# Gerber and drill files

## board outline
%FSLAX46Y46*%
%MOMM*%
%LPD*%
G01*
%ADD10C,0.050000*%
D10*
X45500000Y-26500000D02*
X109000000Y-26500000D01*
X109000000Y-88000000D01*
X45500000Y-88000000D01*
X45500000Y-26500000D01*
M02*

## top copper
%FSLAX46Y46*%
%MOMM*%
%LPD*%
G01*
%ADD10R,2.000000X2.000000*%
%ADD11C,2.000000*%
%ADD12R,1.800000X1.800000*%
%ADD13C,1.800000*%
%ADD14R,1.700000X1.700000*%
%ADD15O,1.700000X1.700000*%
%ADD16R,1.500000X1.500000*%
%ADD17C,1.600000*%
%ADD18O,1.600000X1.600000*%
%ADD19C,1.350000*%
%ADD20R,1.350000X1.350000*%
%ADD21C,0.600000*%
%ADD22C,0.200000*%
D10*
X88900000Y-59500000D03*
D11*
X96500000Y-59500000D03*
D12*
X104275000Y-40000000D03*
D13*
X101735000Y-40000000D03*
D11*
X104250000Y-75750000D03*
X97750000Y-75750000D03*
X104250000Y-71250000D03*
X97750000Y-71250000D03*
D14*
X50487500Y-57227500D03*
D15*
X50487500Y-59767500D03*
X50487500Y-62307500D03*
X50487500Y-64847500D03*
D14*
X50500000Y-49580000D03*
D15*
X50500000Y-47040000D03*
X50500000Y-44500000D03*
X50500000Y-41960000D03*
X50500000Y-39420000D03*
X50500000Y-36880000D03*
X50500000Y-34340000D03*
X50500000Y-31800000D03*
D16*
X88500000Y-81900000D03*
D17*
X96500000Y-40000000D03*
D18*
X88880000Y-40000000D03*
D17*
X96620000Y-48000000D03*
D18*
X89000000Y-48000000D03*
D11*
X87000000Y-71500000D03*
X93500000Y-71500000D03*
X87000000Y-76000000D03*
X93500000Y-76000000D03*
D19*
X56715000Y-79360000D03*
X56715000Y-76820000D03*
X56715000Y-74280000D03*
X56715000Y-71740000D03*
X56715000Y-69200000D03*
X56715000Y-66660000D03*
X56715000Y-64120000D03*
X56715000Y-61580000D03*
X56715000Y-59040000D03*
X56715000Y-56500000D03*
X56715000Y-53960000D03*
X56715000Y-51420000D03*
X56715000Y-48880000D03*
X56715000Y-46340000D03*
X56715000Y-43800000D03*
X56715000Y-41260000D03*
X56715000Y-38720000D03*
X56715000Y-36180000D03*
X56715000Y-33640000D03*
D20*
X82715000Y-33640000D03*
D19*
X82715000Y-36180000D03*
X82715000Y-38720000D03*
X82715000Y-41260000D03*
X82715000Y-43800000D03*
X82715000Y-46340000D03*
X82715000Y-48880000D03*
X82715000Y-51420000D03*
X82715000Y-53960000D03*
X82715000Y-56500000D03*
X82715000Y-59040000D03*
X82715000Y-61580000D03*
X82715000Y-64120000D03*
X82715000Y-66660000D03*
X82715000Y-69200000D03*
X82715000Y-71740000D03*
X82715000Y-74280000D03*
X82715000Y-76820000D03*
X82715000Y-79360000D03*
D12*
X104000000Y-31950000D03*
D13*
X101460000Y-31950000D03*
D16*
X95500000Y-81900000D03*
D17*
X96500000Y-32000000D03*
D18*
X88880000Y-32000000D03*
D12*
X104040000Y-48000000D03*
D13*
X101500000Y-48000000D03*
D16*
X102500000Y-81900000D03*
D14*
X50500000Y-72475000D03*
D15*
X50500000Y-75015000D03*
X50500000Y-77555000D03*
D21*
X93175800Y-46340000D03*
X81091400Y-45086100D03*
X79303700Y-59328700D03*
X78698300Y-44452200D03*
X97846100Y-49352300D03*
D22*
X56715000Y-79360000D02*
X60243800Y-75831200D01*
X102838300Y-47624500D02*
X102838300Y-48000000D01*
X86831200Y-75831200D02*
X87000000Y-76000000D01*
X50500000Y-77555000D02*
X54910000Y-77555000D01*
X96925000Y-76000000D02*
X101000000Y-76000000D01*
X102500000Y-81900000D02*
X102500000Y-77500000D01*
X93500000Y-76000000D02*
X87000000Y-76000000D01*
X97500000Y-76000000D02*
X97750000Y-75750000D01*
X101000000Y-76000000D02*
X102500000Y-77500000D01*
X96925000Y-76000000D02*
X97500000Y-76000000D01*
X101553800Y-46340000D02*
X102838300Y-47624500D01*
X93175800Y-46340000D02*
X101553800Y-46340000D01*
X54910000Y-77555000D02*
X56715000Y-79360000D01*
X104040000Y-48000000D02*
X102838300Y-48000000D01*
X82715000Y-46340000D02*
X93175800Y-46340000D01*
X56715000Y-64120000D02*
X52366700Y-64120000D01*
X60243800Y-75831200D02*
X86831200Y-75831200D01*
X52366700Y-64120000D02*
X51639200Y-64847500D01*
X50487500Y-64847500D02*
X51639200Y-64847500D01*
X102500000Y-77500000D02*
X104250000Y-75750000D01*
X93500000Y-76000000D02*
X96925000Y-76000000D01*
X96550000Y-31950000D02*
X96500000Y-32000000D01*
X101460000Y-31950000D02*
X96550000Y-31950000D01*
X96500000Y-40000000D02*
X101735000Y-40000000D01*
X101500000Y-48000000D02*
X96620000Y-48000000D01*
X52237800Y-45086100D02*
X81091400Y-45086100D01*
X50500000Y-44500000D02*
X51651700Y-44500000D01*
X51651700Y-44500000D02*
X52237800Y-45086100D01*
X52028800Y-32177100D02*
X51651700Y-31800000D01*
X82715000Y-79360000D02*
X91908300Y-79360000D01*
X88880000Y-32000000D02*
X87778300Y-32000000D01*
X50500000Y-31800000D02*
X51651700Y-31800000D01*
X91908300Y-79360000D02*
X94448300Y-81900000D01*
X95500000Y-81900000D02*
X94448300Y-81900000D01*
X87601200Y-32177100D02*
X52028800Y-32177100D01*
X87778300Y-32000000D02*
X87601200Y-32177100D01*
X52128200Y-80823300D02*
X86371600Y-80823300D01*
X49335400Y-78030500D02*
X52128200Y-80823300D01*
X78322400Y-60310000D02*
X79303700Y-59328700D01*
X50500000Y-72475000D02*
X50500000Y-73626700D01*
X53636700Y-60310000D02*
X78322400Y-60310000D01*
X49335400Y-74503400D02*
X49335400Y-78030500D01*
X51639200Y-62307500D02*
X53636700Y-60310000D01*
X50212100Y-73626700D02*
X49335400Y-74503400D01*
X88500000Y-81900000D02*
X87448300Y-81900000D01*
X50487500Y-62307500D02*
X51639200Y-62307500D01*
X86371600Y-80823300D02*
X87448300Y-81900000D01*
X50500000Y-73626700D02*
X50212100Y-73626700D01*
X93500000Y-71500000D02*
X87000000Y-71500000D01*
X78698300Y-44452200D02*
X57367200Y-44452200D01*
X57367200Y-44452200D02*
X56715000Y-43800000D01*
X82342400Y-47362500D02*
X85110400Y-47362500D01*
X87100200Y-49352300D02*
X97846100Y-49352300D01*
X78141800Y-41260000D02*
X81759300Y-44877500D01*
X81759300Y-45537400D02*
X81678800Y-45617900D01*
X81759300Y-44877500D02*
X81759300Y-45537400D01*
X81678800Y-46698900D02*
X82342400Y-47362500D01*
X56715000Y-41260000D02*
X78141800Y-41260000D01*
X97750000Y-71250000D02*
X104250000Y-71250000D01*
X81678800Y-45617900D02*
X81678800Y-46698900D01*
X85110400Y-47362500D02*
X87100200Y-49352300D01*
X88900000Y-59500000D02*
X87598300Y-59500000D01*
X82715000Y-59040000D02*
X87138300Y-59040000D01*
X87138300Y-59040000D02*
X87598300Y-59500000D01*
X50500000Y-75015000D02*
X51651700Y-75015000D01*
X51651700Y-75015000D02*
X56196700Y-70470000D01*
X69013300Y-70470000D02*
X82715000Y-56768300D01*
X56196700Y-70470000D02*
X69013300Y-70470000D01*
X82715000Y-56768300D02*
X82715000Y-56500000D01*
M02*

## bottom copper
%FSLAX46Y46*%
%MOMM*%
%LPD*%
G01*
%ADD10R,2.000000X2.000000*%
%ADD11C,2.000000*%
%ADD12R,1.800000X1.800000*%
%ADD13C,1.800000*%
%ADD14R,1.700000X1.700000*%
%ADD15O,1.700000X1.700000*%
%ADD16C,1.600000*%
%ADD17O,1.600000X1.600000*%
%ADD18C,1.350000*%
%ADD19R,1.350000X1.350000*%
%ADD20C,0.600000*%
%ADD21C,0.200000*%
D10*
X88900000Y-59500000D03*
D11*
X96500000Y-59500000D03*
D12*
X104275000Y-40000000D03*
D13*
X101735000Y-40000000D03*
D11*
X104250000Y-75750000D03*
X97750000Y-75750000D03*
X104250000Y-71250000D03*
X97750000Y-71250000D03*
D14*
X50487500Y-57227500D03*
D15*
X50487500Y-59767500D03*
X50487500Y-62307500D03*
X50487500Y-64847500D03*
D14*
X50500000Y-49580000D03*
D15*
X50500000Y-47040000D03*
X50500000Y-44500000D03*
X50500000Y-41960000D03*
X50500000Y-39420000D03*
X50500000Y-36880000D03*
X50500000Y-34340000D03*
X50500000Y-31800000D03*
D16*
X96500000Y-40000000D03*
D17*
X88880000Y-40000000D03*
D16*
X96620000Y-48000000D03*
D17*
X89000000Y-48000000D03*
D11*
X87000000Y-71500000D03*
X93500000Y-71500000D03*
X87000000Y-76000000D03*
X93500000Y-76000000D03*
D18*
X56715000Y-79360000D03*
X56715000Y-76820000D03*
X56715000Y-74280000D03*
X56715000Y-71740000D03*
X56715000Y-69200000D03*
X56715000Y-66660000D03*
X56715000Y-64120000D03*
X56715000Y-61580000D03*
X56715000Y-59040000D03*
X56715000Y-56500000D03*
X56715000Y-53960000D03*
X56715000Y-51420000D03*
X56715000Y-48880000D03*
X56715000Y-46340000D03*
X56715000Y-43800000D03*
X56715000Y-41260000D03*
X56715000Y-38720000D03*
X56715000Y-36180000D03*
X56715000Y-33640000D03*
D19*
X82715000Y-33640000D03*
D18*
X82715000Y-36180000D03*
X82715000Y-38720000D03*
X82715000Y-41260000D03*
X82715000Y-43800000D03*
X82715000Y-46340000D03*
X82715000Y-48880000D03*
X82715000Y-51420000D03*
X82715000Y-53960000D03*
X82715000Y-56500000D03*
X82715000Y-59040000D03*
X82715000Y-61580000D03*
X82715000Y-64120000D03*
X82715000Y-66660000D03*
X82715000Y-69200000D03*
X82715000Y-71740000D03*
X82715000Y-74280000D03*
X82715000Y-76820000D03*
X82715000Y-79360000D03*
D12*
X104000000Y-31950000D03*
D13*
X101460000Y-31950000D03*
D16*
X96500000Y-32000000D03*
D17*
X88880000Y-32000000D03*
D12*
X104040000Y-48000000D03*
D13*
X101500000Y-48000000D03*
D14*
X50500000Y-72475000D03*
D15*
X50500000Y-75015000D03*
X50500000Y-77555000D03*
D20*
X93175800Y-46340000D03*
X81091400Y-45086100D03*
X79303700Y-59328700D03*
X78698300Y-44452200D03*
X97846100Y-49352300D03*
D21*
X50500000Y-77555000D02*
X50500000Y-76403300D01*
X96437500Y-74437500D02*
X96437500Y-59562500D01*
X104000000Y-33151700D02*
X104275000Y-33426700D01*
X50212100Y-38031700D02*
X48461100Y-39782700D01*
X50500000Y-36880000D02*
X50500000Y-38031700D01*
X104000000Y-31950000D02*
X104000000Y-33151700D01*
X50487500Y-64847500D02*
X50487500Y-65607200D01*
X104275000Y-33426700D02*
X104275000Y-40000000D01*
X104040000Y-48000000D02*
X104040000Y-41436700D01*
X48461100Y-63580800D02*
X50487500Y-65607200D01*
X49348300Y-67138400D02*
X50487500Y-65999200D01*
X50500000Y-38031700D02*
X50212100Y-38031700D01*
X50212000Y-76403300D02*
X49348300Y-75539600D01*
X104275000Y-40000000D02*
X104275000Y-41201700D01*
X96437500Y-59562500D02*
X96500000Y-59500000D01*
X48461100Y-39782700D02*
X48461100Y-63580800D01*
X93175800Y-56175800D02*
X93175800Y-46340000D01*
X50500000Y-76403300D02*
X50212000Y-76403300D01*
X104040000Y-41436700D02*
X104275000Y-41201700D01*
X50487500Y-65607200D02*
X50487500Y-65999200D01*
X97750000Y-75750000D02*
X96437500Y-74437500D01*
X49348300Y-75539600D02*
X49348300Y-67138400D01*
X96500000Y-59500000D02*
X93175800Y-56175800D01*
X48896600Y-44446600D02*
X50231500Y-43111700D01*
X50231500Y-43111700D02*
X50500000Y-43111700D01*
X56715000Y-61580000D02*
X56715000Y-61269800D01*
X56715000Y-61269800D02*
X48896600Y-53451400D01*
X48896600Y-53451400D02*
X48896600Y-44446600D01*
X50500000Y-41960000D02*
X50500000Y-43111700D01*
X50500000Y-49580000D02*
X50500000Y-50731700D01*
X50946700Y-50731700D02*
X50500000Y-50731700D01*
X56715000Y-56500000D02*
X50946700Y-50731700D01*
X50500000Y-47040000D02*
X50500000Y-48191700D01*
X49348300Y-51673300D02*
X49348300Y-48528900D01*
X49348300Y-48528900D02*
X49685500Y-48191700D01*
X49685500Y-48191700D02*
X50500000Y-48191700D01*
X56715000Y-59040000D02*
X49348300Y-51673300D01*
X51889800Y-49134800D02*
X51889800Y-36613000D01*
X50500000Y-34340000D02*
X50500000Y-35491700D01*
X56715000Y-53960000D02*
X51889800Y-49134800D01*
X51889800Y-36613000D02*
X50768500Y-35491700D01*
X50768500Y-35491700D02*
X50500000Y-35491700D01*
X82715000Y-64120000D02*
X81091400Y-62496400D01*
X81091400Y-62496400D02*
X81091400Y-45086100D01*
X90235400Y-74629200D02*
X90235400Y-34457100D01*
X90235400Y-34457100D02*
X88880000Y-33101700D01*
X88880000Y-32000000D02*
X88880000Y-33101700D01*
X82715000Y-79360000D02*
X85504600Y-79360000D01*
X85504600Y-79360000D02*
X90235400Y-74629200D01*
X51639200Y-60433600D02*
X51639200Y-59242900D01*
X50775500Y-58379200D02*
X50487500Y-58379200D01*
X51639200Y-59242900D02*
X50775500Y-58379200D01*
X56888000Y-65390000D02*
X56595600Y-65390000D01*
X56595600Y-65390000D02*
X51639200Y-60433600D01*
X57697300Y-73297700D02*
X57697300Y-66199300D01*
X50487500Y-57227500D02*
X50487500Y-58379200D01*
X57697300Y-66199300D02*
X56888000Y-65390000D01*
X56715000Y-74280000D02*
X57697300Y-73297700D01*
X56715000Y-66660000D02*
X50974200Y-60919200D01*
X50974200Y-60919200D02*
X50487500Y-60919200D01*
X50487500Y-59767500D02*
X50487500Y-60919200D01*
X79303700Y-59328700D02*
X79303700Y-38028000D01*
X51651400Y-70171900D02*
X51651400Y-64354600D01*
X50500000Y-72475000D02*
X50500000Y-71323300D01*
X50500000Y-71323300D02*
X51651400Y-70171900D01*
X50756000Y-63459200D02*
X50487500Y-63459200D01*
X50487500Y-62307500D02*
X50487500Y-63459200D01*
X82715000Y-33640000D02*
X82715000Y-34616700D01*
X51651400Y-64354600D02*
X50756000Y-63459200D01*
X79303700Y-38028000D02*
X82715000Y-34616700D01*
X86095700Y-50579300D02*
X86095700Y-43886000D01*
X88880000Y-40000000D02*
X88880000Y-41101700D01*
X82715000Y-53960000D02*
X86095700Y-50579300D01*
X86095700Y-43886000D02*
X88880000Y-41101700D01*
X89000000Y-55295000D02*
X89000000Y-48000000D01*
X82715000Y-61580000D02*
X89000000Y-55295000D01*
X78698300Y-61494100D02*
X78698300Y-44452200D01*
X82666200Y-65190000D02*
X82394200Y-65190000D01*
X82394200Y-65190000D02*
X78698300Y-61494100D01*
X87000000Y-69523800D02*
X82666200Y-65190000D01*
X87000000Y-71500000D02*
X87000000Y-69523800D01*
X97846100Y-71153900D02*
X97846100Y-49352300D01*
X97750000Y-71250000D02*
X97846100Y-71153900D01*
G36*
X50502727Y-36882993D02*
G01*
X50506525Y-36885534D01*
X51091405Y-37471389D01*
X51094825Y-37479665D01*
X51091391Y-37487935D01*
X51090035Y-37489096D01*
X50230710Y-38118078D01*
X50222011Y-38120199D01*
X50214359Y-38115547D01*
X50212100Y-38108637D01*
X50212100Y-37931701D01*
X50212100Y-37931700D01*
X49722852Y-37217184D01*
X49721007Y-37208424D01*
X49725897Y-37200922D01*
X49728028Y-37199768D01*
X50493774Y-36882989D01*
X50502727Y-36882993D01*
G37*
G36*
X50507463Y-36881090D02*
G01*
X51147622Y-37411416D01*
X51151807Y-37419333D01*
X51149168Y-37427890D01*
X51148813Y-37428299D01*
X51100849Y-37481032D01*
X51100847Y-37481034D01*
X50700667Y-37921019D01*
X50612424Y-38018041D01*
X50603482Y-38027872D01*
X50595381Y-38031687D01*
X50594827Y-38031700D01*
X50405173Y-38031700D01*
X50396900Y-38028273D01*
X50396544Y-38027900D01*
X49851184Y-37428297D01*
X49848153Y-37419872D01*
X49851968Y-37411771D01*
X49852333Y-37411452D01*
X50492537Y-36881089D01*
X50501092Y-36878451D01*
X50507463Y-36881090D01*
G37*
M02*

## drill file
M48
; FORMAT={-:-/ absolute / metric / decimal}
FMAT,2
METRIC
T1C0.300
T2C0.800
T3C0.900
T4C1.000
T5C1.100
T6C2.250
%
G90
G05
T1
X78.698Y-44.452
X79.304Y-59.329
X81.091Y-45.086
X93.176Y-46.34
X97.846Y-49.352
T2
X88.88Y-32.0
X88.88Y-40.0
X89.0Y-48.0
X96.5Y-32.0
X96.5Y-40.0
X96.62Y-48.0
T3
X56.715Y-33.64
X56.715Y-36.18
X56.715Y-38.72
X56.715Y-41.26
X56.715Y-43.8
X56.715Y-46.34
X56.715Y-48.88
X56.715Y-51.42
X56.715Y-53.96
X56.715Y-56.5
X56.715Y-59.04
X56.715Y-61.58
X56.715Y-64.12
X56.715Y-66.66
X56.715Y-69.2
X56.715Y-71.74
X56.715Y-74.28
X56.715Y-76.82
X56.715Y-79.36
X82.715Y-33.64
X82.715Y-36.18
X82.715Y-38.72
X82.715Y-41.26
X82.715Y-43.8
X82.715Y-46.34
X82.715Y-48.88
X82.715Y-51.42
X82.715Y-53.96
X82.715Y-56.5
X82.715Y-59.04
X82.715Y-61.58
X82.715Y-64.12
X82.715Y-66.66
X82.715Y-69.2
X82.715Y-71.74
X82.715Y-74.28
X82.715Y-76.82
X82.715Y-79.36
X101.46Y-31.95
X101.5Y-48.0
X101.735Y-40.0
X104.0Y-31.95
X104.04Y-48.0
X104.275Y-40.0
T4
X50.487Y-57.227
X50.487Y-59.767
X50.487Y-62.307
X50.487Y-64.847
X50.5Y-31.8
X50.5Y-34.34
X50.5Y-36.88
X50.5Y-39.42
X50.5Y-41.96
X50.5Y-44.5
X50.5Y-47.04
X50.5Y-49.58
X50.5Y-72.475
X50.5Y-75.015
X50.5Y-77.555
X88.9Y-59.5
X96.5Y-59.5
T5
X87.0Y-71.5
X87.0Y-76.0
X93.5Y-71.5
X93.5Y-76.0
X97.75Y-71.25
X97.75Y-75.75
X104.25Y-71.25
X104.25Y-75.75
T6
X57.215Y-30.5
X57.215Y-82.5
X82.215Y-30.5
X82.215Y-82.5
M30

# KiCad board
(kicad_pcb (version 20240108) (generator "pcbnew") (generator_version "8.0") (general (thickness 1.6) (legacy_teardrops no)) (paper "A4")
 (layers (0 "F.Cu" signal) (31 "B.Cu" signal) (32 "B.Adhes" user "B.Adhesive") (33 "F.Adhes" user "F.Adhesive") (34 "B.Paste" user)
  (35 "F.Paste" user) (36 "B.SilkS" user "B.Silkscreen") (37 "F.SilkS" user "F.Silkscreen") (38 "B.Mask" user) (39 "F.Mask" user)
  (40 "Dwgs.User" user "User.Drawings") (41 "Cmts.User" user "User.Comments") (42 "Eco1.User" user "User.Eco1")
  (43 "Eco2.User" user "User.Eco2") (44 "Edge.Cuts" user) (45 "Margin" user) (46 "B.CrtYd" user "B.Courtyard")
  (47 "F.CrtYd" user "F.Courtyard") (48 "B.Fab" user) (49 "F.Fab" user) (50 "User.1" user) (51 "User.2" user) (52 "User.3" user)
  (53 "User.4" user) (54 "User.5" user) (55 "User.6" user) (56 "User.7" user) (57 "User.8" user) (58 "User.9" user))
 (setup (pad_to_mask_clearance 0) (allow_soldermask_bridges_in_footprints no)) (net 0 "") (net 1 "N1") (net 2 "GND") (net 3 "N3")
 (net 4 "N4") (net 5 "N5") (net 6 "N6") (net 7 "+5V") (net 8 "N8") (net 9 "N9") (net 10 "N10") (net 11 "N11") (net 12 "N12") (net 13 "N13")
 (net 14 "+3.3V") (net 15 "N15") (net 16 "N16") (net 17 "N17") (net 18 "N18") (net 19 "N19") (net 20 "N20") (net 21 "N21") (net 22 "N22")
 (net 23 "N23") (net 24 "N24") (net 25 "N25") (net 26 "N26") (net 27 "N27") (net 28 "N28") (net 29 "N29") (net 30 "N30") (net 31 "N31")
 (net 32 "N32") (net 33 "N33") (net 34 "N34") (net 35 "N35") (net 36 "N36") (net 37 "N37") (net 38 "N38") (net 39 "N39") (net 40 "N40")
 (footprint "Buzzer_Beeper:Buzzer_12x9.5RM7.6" (layer "F.Cu") (at 88.9 59.5)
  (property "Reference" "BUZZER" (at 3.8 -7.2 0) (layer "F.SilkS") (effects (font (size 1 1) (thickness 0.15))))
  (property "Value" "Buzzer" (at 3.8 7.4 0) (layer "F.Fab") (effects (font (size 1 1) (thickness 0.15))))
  (pad "1" thru_hole rect (at 0 0) (size 2 2) (drill 1) (layers "*.Cu" "*.Mask") (remove_unused_layers no) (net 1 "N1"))
  (pad "2" thru_hole circle (at 7.6 0) (size 2 2) (drill 1) (layers "*.Cu" "*.Mask") (remove_unused_layers no) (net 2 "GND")))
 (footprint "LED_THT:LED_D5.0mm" (layer "F.Cu") (at 104.275 40 180)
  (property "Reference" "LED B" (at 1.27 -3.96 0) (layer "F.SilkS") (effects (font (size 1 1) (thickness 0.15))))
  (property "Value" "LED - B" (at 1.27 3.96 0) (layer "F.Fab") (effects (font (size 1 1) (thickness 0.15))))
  (pad "1" thru_hole rect (at 0 0 180) (size 1.8 1.8) (drill 0.9) (layers "*.Cu" "*.Mask") (remove_unused_layers no) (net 2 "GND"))
  (pad "2" thru_hole circle (at 2.54 0 180) (size 1.8 1.8) (drill 0.9) (layers "*.Cu" "*.Mask") (remove_unused_layers no) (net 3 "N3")))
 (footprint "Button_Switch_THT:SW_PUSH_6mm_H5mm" (layer "F.Cu") (at 104.25 75.75 180)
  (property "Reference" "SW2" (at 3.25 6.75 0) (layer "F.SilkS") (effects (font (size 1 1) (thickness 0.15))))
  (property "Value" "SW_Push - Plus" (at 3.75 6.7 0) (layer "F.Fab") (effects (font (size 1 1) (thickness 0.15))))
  (pad "1" thru_hole circle (at 0 0 270) (size 2 2) (drill 1.1) (layers "*.Cu" "*.Mask") (remove_unused_layers no) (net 2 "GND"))
  (pad "1" thru_hole circle (at 6.5 0 270) (size 2 2) (drill 1.1) (layers "*.Cu" "*.Mask") (remove_unused_layers no) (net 2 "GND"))
  (pad "2" thru_hole circle (at 0 4.5 270) (size 2 2) (drill 1.1) (layers "*.Cu" "*.Mask") (remove_unused_layers no) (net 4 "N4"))
  (pad "2" thru_hole circle (at 6.5 4.5 270) (size 2 2) (drill 1.1) (layers "*.Cu" "*.Mask") (remove_unused_layers no) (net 4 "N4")))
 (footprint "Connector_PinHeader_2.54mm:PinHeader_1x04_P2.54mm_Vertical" (layer "F.Cu") (at 50.4875 57.2275)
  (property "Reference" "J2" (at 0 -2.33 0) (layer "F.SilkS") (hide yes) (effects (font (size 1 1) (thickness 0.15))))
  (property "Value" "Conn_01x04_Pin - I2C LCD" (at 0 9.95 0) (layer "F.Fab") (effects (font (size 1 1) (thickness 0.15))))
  (pad "1" thru_hole rect (at 0 0) (size 1.7 1.7) (drill 1) (layers "*.Cu" "*.Mask") (remove_unused_layers no) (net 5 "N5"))
  (pad "2" thru_hole oval (at 0 2.54) (size 1.7 1.7) (drill 1) (layers "*.Cu" "*.Mask") (remove_unused_layers no) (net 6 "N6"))
  (pad "3" thru_hole oval (at 0 5.08) (size 1.7 1.7) (drill 1) (layers "*.Cu" "*.Mask") (remove_unused_layers no) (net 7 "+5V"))
  (pad "4" thru_hole oval (at 0 7.62) (size 1.7 1.7) (drill 1) (layers "*.Cu" "*.Mask") (remove_unused_layers no) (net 2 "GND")))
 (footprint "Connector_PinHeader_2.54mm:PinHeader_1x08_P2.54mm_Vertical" (layer "F.Cu") (at 50.5 49.58 180)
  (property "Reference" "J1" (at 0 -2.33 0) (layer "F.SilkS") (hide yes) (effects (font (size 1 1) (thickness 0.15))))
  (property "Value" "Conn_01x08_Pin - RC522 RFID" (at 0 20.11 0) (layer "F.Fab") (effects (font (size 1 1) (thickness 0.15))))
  (pad "1" thru_hole rect (at 0 0 180) (size 1.7 1.7) (drill 1) (layers "*.Cu" "*.Mask") (remove_unused_layers no) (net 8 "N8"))
  (pad "2" thru_hole oval (at 0 2.54 180) (size 1.7 1.7) (drill 1) (layers "*.Cu" "*.Mask") (remove_unused_layers no) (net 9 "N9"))
  (pad "3" thru_hole oval (at 0 5.08 180) (size 1.7 1.7) (drill 1) (layers "*.Cu" "*.Mask") (remove_unused_layers no) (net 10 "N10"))
  (pad "4" thru_hole oval (at 0 7.62 180) (size 1.7 1.7) (drill 1) (layers "*.Cu" "*.Mask") (remove_unused_layers no) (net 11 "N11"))
  (pad "5" thru_hole oval (at 0 10.16 180) (size 1.7 1.7) (drill 1) (layers "*.Cu" "*.Mask") (remove_unused_layers no) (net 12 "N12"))
  (pad "6" thru_hole oval (at 0 12.7 180) (size 1.7 1.7) (drill 1) (layers "*.Cu" "*.Mask") (remove_unused_layers no) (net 2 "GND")
   (teardrops (best_length_ratio 0.5) (max_length 1) (best_width_ratio 1) (max_width 2) (curve_points 0) (filter_ratio 0.9) (enabled yes)
    (allow_two_segments yes) (prefer_zone_connections yes)))
  (pad "7" thru_hole oval (at 0 15.24 180) (size 1.7 1.7) (drill 1) (layers "*.Cu" "*.Mask") (remove_unused_layers no) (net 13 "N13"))
  (pad "8" thru_hole oval (at 0 17.78 180) (size 1.7 1.7) (drill 1) (layers "*.Cu" "*.Mask") (remove_unused_layers no) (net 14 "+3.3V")))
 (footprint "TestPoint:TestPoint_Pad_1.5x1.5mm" (layer "F.Cu") (at 88.5 81.9 -90)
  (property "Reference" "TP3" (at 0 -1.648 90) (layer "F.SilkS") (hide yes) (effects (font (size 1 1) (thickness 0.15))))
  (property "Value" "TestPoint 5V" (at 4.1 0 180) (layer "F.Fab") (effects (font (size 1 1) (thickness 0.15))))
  (pad "1" smd rect (at 0 0 270) (size 1.5 1.5) (layers "F.Cu" "F.Mask") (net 7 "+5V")))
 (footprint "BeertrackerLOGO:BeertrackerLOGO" (layer "F.Cu") (at 102.5 59.5 90)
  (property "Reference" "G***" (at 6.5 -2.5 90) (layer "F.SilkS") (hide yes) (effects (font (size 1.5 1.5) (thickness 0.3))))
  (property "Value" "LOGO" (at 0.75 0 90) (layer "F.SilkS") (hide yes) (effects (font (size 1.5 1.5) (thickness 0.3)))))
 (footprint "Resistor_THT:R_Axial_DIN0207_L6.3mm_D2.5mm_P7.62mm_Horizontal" (layer "F.Cu") (at 96.5 40 180)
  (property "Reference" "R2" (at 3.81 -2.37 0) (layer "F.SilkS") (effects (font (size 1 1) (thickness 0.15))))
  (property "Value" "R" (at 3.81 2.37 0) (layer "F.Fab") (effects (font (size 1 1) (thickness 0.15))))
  (pad "1" thru_hole circle (at 0 0 180) (size 1.6 1.6) (drill 0.8) (layers "*.Cu" "*.Mask") (remove_unused_layers no) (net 3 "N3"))
  (pad "2" thru_hole oval (at 7.62 0 180) (size 1.6 1.6) (drill 0.8) (layers "*.Cu" "*.Mask") (remove_unused_layers no) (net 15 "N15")))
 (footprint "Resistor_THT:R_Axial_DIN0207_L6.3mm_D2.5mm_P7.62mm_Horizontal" (layer "F.Cu") (at 96.62 48 180)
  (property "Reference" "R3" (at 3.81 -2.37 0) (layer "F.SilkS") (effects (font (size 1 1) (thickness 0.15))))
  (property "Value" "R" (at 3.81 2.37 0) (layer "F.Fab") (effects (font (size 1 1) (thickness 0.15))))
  (pad "1" thru_hole circle (at 0 0 180) (size 1.6 1.6) (drill 0.8) (layers "*.Cu" "*.Mask") (remove_unused_layers no) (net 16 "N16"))
  (pad "2" thru_hole oval (at 7.62 0 180) (size 1.6 1.6) (drill 0.8) (layers "*.Cu" "*.Mask") (remove_unused_layers no) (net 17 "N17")))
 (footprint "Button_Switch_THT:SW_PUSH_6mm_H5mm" (layer "F.Cu") (at 87 71.5)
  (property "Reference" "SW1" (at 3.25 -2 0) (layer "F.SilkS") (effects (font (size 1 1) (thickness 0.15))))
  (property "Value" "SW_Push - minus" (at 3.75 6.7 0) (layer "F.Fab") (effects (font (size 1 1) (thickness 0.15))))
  (pad "1" thru_hole circle (at 0 0 90) (size 2 2) (drill 1.1) (layers "*.Cu" "*.Mask") (remove_unused_layers no) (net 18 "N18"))
  (pad "1" thru_hole circle (at 6.5 0 90) (size 2 2) (drill 1.1) (layers "*.Cu" "*.Mask") (remove_unused_layers no) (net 18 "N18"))
  (pad "2" thru_hole circle (at 0 4.5 90) (size 2 2) (drill 1.1) (layers "*.Cu" "*.Mask") (remove_unused_layers no) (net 2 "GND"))
  (pad "2" thru_hole circle (at 6.5 4.5 90) (size 2 2) (drill 1.1) (layers "*.Cu" "*.Mask") (remove_unused_layers no) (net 2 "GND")))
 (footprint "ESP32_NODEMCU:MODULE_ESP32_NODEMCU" (layer "F.Cu") (at 69.715 56.5 180)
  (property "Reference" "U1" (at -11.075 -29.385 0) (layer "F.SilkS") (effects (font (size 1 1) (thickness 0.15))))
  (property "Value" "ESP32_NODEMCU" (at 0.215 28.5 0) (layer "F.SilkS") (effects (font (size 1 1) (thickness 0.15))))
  (pad "" np_thru_hole circle (at -12.5 -26 180) (size 2.25 2.25) (drill 2.25) (layers "*.Cu" "*.Mask"))
  (pad "" np_thru_hole circle (at -12.5 26 180) (size 2.25 2.25) (drill 2.25) (layers "*.Cu" "*.Mask"))
  (pad "" np_thru_hole circle (at 12.5 -26 180) (size 2.25 2.25) (drill 2.25) (layers "*.Cu" "*.Mask"))
  (pad "" np_thru_hole circle (at 12.5 26 180) (size 2.25 2.25) (drill 2.25) (layers "*.Cu" "*.Mask"))
  (pad "J4_1" thru_hole circle (at 13 -22.86 180) (size 1.35 1.35) (drill 0.9) (layers "*.Cu" "*.Mask") (remove_unused_layers no)
   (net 2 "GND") (solder_mask_margin 0.102))
  (pad "J4_2" thru_hole circle (at 13 -20.32 180) (size 1.35 1.35) (drill 0.9) (layers "*.Cu" "*.Mask") (remove_unused_layers no)
   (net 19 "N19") (solder_mask_margin 0.102))
  (pad "J4_3" thru_hole circle (at 13 -17.78 180) (size 1.35 1.35) (drill 0.9) (layers "*.Cu" "*.Mask") (remove_unused_layers no)
   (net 5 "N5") (solder_mask_margin 0.102))
  (pad "J4_4" thru_hole circle (at 13 -15.24 180) (size 1.35 1.35) (drill 0.9) (layers "*.Cu" "*.Mask") (remove_unused_layers no)
   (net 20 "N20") (solder_mask_margin 0.102))
  (pad "J4_5" thru_hole circle (at 13 -12.7 180) (size 1.35 1.35) (drill 0.9) (layers "*.Cu" "*.Mask") (remove_unused_layers no)
   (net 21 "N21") (solder_mask_margin 0.102))
  (pad "J4_6" thru_hole circle (at 13 -10.16 180) (size 1.35 1.35) (drill 0.9) (layers "*.Cu" "*.Mask") (remove_unused_layers no)
   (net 6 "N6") (solder_mask_margin 0.102))
  (pad "J4_7" thru_hole circle (at 13 -7.62 180) (size 1.35 1.35) (drill 0.9) (layers "*.Cu" "*.Mask") (remove_unused_layers no)
   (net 2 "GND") (solder_mask_margin 0.102))
  (pad "J4_8" thru_hole circle (at 13 -5.08 180) (size 1.35 1.35) (drill 0.9) (layers "*.Cu" "*.Mask") (remove_unused_layers no)
   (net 11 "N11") (solder_mask_margin 0.102))
  (pad "J4_9" thru_hole circle (at 13 -2.54 180) (size 1.35 1.35) (drill 0.9) (layers "*.Cu" "*.Mask") (remove_unused_layers no)
   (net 9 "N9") (solder_mask_margin 0.102))
  (pad "J4_10" thru_hole circle (at 13 0 180) (size 1.35 1.35) (drill 0.9) (layers "*.Cu" "*.Mask") (remove_unused_layers no) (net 8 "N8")
   (solder_mask_margin 0.102))
  (pad "J4_11" thru_hole circle (at 13 2.54 180) (size 1.35 1.35) (drill 0.9) (layers "*.Cu" "*.Mask") (remove_unused_layers no)
   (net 13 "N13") (solder_mask_margin 0.102))
  (pad "J4_12" thru_hole circle (at 13 5.08 180) (size 1.35 1.35) (drill 0.9) (layers "*.Cu" "*.Mask") (remove_unused_layers no)
   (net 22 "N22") (solder_mask_margin 0.102))
  (pad "J4_13" thru_hole circle (at 13 7.62 180) (size 1.35 1.35) (drill 0.9) (layers "*.Cu" "*.Mask") (remove_unused_layers no)
   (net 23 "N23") (solder_mask_margin 0.102))
  (pad "J4_14" thru_hole circle (at 13 10.16 180) (size 1.35 1.35) (drill 0.9) (layers "*.Cu" "*.Mask") (remove_unused_layers no)
   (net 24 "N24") (solder_mask_margin 0.102))
  (pad "J4_15" thru_hole circle (at 13 12.7 180) (size 1.35 1.35) (drill 0.9) (layers "*.Cu" "*.Mask") (remove_unused_layers no)
   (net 18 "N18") (solder_mask_margin 0.102))
  (pad "J4_16" thru_hole circle (at 13 15.24 180) (size 1.35 1.35) (drill 0.9) (layers "*.Cu" "*.Mask") (remove_unused_layers no)
   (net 4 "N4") (solder_mask_margin 0.102))
  (pad "J4_17" thru_hole circle (at 13 17.78 180) (size 1.35 1.35) (drill 0.9) (layers "*.Cu" "*.Mask") (remove_unused_layers no)
   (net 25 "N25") (solder_mask_margin 0.102))
  (pad "J4_18" thru_hole circle (at 13 20.32 180) (size 1.35 1.35) (drill 0.9) (layers "*.Cu" "*.Mask") (remove_unused_layers no)
   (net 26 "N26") (solder_mask_margin 0.102))
  (pad "J4_19" thru_hole circle (at 13 22.86 180) (size 1.35 1.35) (drill 0.9) (layers "*.Cu" "*.Mask") (remove_unused_layers no)
   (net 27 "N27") (solder_mask_margin 0.102))
  (pad "J5_1" thru_hole rect (at -13 22.86 180) (size 1.35 1.35) (drill 0.9) (layers "*.Cu" "*.Mask") (remove_unused_layers no)
   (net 7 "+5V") (solder_mask_margin 0.102))
  (pad "J5_2" thru_hole circle (at -13 20.32 180) (size 1.35 1.35) (drill 0.9) (layers "*.Cu" "*.Mask") (remove_unused_layers no)
   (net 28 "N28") (solder_mask_margin 0.102))
  (pad "J5_3" thru_hole circle (at -13 17.78 180) (size 1.35 1.35) (drill 0.9) (layers "*.Cu" "*.Mask") (remove_unused_layers no)
   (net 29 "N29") (solder_mask_margin 0.102))
  (pad "J5_4" thru_hole circle (at -13 15.24 180) (size 1.35 1.35) (drill 0.9) (layers "*.Cu" "*.Mask") (remove_unused_layers no)
   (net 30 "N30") (solder_mask_margin 0.102))
  (pad "J5_5" thru_hole circle (at -13 12.7 180) (size 1.35 1.35) (drill 0.9) (layers "*.Cu" "*.Mask") (remove_unused_layers no)
   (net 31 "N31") (solder_mask_margin 0.102))
  (pad "J5_6" thru_hole circle (at -13 10.16 180) (size 1.35 1.35) (drill 0.9) (layers "*.Cu" "*.Mask") (remove_unused_layers no)
   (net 2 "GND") (solder_mask_margin 0.102))
  (pad "J5_7" thru_hole circle (at -13 7.62 180) (size 1.35 1.35) (drill 0.9) (layers "*.Cu" "*.Mask") (remove_unused_layers no)
   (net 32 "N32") (solder_mask_margin 0.102))
  (pad "J5_8" thru_hole circle (at -13 5.08 180) (size 1.35 1.35) (drill 0.9) (layers "*.Cu" "*.Mask") (remove_unused_layers no)
   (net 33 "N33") (solder_mask_margin 0.102))
  (pad "J5_9" thru_hole circle (at -13 2.54 180) (size 1.35 1.35) (drill 0.9) (layers "*.Cu" "*.Mask") (remove_unused_layers no)
   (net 15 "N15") (solder_mask_margin 0.102))
  (pad "J5_10" thru_hole circle (at -13 0 180) (size 1.35 1.35) (drill 0.9) (layers "*.Cu" "*.Mask") (remove_unused_layers no)
   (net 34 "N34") (solder_mask_margin 0.102))
  (pad "J5_11" thru_hole circle (at -13 -2.54 180) (size 1.35 1.35) (drill 0.9) (layers "*.Cu" "*.Mask") (remove_unused_layers no)
   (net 1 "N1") (solder_mask_margin 0.102))
  (pad "J5_12" thru_hole circle (at -13 -5.08 180) (size 1.35 1.35) (drill 0.9) (layers "*.Cu" "*.Mask") (remove_unused_layers no)
   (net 17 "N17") (solder_mask_margin 0.102))
  (pad "J5_13" thru_hole circle (at -13 -7.62 180) (size 1.35 1.35) (drill 0.9) (layers "*.Cu" "*.Mask") (remove_unused_layers no)
   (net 10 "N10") (solder_mask_margin 0.102))
  (pad "J5_14" thru_hole circle (at -13 -10.16 180) (size 1.35 1.35) (drill 0.9) (layers "*.Cu" "*.Mask") (remove_unused_layers no)
   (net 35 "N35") (solder_mask_margin 0.102))
  (pad "J5_15" thru_hole circle (at -13 -12.7 180) (size 1.35 1.35) (drill 0.9) (layers "*.Cu" "*.Mask") (remove_unused_layers no)
   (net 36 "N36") (solder_mask_margin 0.102))
  (pad "J5_16" thru_hole circle (at -13 -15.24 180) (size 1.35 1.35) (drill 0.9) (layers "*.Cu" "*.Mask") (remove_unused_layers no)
   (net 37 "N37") (solder_mask_margin 0.102))
  (pad "J5_17" thru_hole circle (at -13 -17.78 180) (size 1.35 1.35) (drill 0.9) (layers "*.Cu" "*.Mask") (remove_unused_layers no)
   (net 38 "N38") (solder_mask_margin 0.102))
  (pad "J5_18" thru_hole circle (at -13 -20.32 180) (size 1.35 1.35) (drill 0.9) (layers "*.Cu" "*.Mask") (remove_unused_layers no)
   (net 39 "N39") (solder_mask_margin 0.102))
  (pad "J5_19" thru_hole circle (at -13 -22.86 180) (size 1.35 1.35) (drill 0.9) (layers "*.Cu" "*.Mask") (remove_unused_layers no)
   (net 14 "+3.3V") (solder_mask_margin 0.102)))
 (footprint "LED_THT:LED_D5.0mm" (layer "F.Cu") (at 104 31.95 180)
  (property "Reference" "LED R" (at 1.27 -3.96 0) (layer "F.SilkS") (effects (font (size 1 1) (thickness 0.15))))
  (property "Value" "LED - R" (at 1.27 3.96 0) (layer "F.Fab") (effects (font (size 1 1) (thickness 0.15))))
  (pad "1" thru_hole rect (at 0 0 180) (size 1.8 1.8) (drill 0.9) (layers "*.Cu" "*.Mask") (remove_unused_layers no) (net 2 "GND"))
  (pad "2" thru_hole circle (at 2.54 0 180) (size 1.8 1.8) (drill 0.9) (layers "*.Cu" "*.Mask") (remove_unused_layers no) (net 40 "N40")))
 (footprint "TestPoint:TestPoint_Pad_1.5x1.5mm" (layer "F.Cu") (at 95.5 81.9 -90)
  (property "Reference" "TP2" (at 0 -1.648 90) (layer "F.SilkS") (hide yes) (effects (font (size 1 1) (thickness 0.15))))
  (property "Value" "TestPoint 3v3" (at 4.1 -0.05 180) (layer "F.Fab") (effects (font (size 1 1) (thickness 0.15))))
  (pad "1" smd rect (at 0 0 270) (size 1.5 1.5) (layers "F.Cu" "F.Mask") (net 14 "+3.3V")))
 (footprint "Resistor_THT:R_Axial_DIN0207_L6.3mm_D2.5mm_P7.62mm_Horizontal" (layer "F.Cu") (at 96.5 32 180)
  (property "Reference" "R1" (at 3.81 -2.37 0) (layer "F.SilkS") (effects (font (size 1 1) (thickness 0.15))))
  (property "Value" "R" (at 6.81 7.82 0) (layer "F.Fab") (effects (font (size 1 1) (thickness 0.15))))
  (pad "1" thru_hole circle (at 0 0 180) (size 1.6 1.6) (drill 0.8) (layers "*.Cu" "*.Mask") (remove_unused_layers no) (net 40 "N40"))
  (pad "2" thru_hole oval (at 7.62 0 180) (size 1.6 1.6) (drill 0.8) (layers "*.Cu" "*.Mask") (remove_unused_layers no) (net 14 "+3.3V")))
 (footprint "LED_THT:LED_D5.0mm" (layer "F.Cu") (at 104.04 48 180)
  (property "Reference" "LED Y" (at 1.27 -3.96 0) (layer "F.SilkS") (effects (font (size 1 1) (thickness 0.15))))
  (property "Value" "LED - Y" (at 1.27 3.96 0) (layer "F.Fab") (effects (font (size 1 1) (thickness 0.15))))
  (pad "1" thru_hole rect (at 0 0 180) (size 1.8 1.8) (drill 0.9) (layers "*.Cu" "*.Mask") (remove_unused_layers no) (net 2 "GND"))
  (pad "2" thru_hole circle (at 2.54 0 180) (size 1.8 1.8) (drill 0.9) (layers "*.Cu" "*.Mask") (remove_unused_layers no) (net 16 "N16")))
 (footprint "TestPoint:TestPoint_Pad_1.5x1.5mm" (layer "F.Cu") (at 102.5 81.9)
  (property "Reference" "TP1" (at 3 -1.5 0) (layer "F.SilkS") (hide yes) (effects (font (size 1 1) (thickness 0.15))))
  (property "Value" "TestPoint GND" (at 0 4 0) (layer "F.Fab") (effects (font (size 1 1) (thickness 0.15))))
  (pad "1" smd rect (at 0 0) (size 1.5 1.5) (layers "F.Cu" "F.Mask") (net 2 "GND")))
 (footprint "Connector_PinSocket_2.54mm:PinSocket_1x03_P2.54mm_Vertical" (layer "F.Cu") (at 50.5 72.475)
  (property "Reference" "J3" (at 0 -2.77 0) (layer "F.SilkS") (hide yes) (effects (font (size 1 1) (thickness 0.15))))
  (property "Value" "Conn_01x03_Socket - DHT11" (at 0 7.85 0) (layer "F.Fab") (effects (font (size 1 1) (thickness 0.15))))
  (pad "1" thru_hole rect (at 0 0) (size 1.7 1.7) (drill 1) (layers "*.Cu" "*.Mask") (remove_unused_layers no) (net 7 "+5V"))
  (pad "2" thru_hole oval (at 0 2.54) (size 1.7 1.7) (drill 1) (layers "*.Cu" "*.Mask") (remove_unused_layers no) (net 34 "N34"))
  (pad "3" thru_hole oval (at 0 5.08) (size 1.7 1.7) (drill 1) (layers "*.Cu" "*.Mask") (remove_unused_layers no) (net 2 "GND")))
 (gr_rect (start 45.5 26.5) (end 109 88) (stroke (width 0.05) (type default)) (fill none) (layer "Edge.Cuts"))
 (segment (start 56.715 79.36) (end 60.2438 75.8312) (width 0.2) (layer "F.Cu") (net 2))
 (segment (start 102.8383 47.6245) (end 102.8383 48) (width 0.2) (layer "F.Cu") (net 2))
 (segment (start 86.8312 75.8312) (end 87 76) (width 0.2) (layer "F.Cu") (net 2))
 (segment (start 50.5 77.555) (end 54.91 77.555) (width 0.2) (layer "F.Cu") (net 2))
 (segment (start 96.925 76) (end 101 76) (width 0.2) (layer "F.Cu") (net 2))
 (segment (start 102.5 81.9) (end 102.5 77.5) (width 0.2) (layer "F.Cu") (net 2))
 (segment (start 93.5 76) (end 87 76) (width 0.2) (layer "F.Cu") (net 2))
 (segment (start 97.5 76) (end 97.75 75.75) (width 0.2) (layer "F.Cu") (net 2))
 (segment (start 101 76) (end 102.5 77.5) (width 0.2) (layer "F.Cu") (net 2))
 (segment (start 96.925 76) (end 97.5 76) (width 0.2) (layer "F.Cu") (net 2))
 (segment (start 101.5538 46.34) (end 102.8383 47.6245) (width 0.2) (layer "F.Cu") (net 2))
 (segment (start 93.1758 46.34) (end 101.5538 46.34) (width 0.2) (layer "F.Cu") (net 2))
 (segment (start 54.91 77.555) (end 56.715 79.36) (width 0.2) (layer "F.Cu") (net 2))
 (segment (start 104.04 48) (end 102.8383 48) (width 0.2) (layer "F.Cu") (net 2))
 (segment (start 82.715 46.34) (end 93.1758 46.34) (width 0.2) (layer "F.Cu") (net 2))
 (segment (start 56.715 64.12) (end 52.3667 64.12) (width 0.2) (layer "F.Cu") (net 2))
 (segment (start 60.2438 75.8312) (end 86.8312 75.8312) (width 0.2) (layer "F.Cu") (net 2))
 (segment (start 52.3667 64.12) (end 51.6392 64.8475) (width 0.2) (layer "F.Cu") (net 2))
 (segment (start 50.4875 64.8475) (end 51.6392 64.8475) (width 0.2) (layer "F.Cu") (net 2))
 (segment (start 102.5 77.5) (end 104.25 75.75) (width 0.2) (layer "F.Cu") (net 2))
 (segment (start 93.5 76) (end 96.925 76) (width 0.2) (layer "F.Cu") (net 2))
 (via (at 93.1758 46.34) (size 0.6) (drill 0.3) (layers "F.Cu" "B.Cu") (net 2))
 (segment (start 50.5 77.555) (end 50.5 76.4033) (width 0.2) (layer "B.Cu") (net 2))
 (segment (start 96.4375 74.4375) (end 96.4375 59.5625) (width 0.2) (layer "B.Cu") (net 2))
 (segment (start 104 33.1517) (end 104.275 33.4267) (width 0.2) (layer "B.Cu") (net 2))
 (segment (start 50.2121 38.0317) (end 48.4611 39.7827) (width 0.2) (layer "B.Cu") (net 2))
 (segment (start 50.5 36.88) (end 50.5 38.0317) (width 0.2) (layer "B.Cu") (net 2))
 (segment (start 104 31.95) (end 104 33.1517) (width 0.2) (layer "B.Cu") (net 2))
 (segment (start 50.4875 64.8475) (end 50.4875 65.6072) (width 0.2) (layer "B.Cu") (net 2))
 (segment (start 104.275 33.4267) (end 104.275 40) (width 0.2) (layer "B.Cu") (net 2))
 (segment (start 104.04 48) (end 104.04 41.4367) (width 0.2) (layer "B.Cu") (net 2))
 (segment (start 48.4611 63.5808) (end 50.4875 65.6072) (width 0.2) (layer "B.Cu") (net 2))
 (segment (start 49.3483 67.1384) (end 50.4875 65.9992) (width 0.2) (layer "B.Cu") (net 2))
 (segment (start 50.5 38.0317) (end 50.2121 38.0317) (width 0.2) (layer "B.Cu") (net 2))
 (segment (start 50.212 76.4033) (end 49.3483 75.5396) (width 0.2) (layer "B.Cu") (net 2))
 (segment (start 104.275 40) (end 104.275 41.2017) (width 0.2) (layer "B.Cu") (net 2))
 (segment (start 96.4375 59.5625) (end 96.5 59.5) (width 0.2) (layer "B.Cu") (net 2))
 (segment (start 48.4611 39.7827) (end 48.4611 63.5808) (width 0.2) (layer "B.Cu") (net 2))
 (segment (start 93.1758 56.1758) (end 93.1758 46.34) (width 0.2) (layer "B.Cu") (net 2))
 (segment (start 50.5 76.4033) (end 50.212 76.4033) (width 0.2) (layer "B.Cu") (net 2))
 (segment (start 104.04 41.4367) (end 104.275 41.2017) (width 0.2) (layer "B.Cu") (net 2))
 (segment (start 50.4875 65.6072) (end 50.4875 65.9992) (width 0.2) (layer "B.Cu") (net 2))
 (segment (start 97.75 75.75) (end 96.4375 74.4375) (width 0.2) (layer "B.Cu") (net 2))
 (segment (start 49.3483 75.5396) (end 49.3483 67.1384) (width 0.2) (layer "B.Cu") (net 2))
 (segment (start 96.5 59.5) (end 93.1758 56.1758) (width 0.2) (layer "B.Cu") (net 2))
 (segment (start 96.55 31.95) (end 96.5 32) (width 0.2) (layer "F.Cu") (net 40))
 (segment (start 101.46 31.95) (end 96.55 31.95) (width 0.2) (layer "F.Cu") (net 40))
 (segment (start 96.5 40) (end 101.735 40) (width 0.2) (layer "F.Cu") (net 3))
 (segment (start 101.5 48) (end 96.62 48) (width 0.2) (layer "F.Cu") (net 16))
 (segment (start 48.8966 44.4466) (end 50.2315 43.1117) (width 0.2) (layer "B.Cu") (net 11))
 (segment (start 50.2315 43.1117) (end 50.5 43.1117) (width 0.2) (layer "B.Cu") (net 11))
 (segment (start 56.715 61.58) (end 56.715 61.2698) (width 0.2) (layer "B.Cu") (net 11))
 (segment (start 56.715 61.2698) (end 48.8966 53.4514) (width 0.2) (layer "B.Cu") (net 11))
 (segment (start 48.8966 53.4514) (end 48.8966 44.4466) (width 0.2) (layer "B.Cu") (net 11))
 (segment (start 50.5 41.96) (end 50.5 43.1117) (width 0.2) (layer "B.Cu") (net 11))
 (segment (start 50.5 49.58) (end 50.5 50.7317) (width 0.2) (layer "B.Cu") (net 8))
 (segment (start 50.9467 50.7317) (end 50.5 50.7317) (width 0.2) (layer "B.Cu") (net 8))
 (segment (start 56.715 56.5) (end 50.9467 50.7317) (width 0.2) (layer "B.Cu") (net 8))
 (segment (start 50.5 47.04) (end 50.5 48.1917) (width 0.2) (layer "B.Cu") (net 9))
 (segment (start 49.3483 51.6733) (end 49.3483 48.5289) (width 0.2) (layer "B.Cu") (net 9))
 (segment (start 49.3483 48.5289) (end 49.6855 48.1917) (width 0.2) (layer "B.Cu") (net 9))
 (segment (start 49.6855 48.1917) (end 50.5 48.1917) (width 0.2) (layer "B.Cu") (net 9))
 (segment (start 56.715 59.04) (end 49.3483 51.6733) (width 0.2) (layer "B.Cu") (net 9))
 (segment (start 51.8898 49.1348) (end 51.8898 36.613) (width 0.2) (layer "B.Cu") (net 13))
 (segment (start 50.5 34.34) (end 50.5 35.4917) (width 0.2) (layer "B.Cu") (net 13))
 (segment (start 56.715 53.96) (end 51.8898 49.1348) (width 0.2) (layer "B.Cu") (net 13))
 (segment (start 51.8898 36.613) (end 50.7685 35.4917) (width 0.2) (layer "B.Cu") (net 13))
 (segment (start 50.7685 35.4917) (end 50.5 35.4917) (width 0.2) (layer "B.Cu") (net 13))
 (segment (start 52.2378 45.0861) (end 81.0914 45.0861) (width 0.2) (layer "F.Cu") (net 10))
 (segment (start 50.5 44.5) (end 51.6517 44.5) (width 0.2) (layer "F.Cu") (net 10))
 (segment (start 51.6517 44.5) (end 52.2378 45.0861) (width 0.2) (layer "F.Cu") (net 10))
 (via (at 81.0914 45.0861) (size 0.6) (drill 0.3) (layers "F.Cu" "B.Cu") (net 10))
 (segment (start 82.715 64.12) (end 81.0914 62.4964) (width 0.2) (layer "B.Cu") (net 10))
 (segment (start 81.0914 62.4964) (end 81.0914 45.0861) (width 0.2) (layer "B.Cu") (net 10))
 (segment (start 52.0288 32.1771) (end 51.6517 31.8) (width 0.2) (layer "F.Cu") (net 14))
 (segment (start 82.715 79.36) (end 91.9083 79.36) (width 0.2) (layer "F.Cu") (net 14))
 (segment (start 88.88 32) (end 87.7783 32) (width 0.2) (layer "F.Cu") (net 14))
 (segment (start 50.5 31.8) (end 51.6517 31.8) (width 0.2) (layer "F.Cu") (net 14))
 (segment (start 91.9083 79.36) (end 94.4483 81.9) (width 0.2) (layer "F.Cu") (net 14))
 (segment (start 95.5 81.9) (end 94.4483 81.9) (width 0.2) (layer "F.Cu") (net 14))
 (segment (start 87.6012 32.1771) (end 52.0288 32.1771) (width 0.2) (layer "F.Cu") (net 14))
 (segment (start 87.7783 32) (end 87.6012 32.1771) (width 0.2) (layer "F.Cu") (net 14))
 (segment (start 90.2354 74.6292) (end 90.2354 34.4571) (width 0.2) (layer "B.Cu") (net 14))
 (segment (start 90.2354 34.4571) (end 88.88 33.1017) (width 0.2) (layer "B.Cu") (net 14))
 (segment (start 88.88 32) (end 88.88 33.1017) (width 0.2) (layer "B.Cu") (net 14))
 (segment (start 82.715 79.36) (end 85.5046 79.36) (width 0.2) (layer "B.Cu") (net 14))
 (segment (start 85.5046 79.36) (end 90.2354 74.6292) (width 0.2) (layer "B.Cu") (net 14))
 (segment (start 51.6392 60.4336) (end 51.6392 59.2429) (width 0.2) (layer "B.Cu") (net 5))
 (segment (start 50.7755 58.3792) (end 50.4875 58.3792) (width 0.2) (layer "B.Cu") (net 5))
 (segment (start 51.6392 59.2429) (end 50.7755 58.3792) (width 0.2) (layer "B.Cu") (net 5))
 (segment (start 56.888 65.39) (end 56.5956 65.39) (width 0.2) (layer "B.Cu") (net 5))
 (segment (start 56.5956 65.39) (end 51.6392 60.4336) (width 0.2) (layer "B.Cu") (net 5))
 (segment (start 57.6973 73.2977) (end 57.6973 66.1993) (width 0.2) (layer "B.Cu") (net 5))
 (segment (start 50.4875 57.2275) (end 50.4875 58.3792) (width 0.2) (layer "B.Cu") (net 5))
 (segment (start 57.6973 66.1993) (end 56.888 65.39) (width 0.2) (layer "B.Cu") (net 5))
 (segment (start 56.715 74.28) (end 57.6973 73.2977) (width 0.2) (layer "B.Cu") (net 5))
 (segment (start 56.715 66.66) (end 50.9742 60.9192) (width 0.2) (layer "B.Cu") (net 6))
 (segment (start 50.9742 60.9192) (end 50.4875 60.9192) (width 0.2) (layer "B.Cu") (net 6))
 (segment (start 50.4875 59.7675) (end 50.4875 60.9192) (width 0.2) (layer "B.Cu") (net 6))
 (segment (start 52.1282 80.8233) (end 86.3716 80.8233) (width 0.2) (layer "F.Cu") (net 7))
 (segment (start 49.3354 78.0305) (end 52.1282 80.8233) (width 0.2) (layer "F.Cu") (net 7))
 (segment (start 78.3224 60.31) (end 79.3037 59.3287) (width 0.2) (layer "F.Cu") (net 7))
 (segment (start 50.5 72.475) (end 50.5 73.6267) (width 0.2) (layer "F.Cu") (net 7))
 (segment (start 53.6367 60.31) (end 78.3224 60.31) (width 0.2) (layer "F.Cu") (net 7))
 (segment (start 49.3354 74.5034) (end 49.3354 78.0305) (width 0.2) (layer "F.Cu") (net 7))
 (segment (start 51.6392 62.3075) (end 53.6367 60.31) (width 0.2) (layer "F.Cu") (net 7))
 (segment (start 50.2121 73.6267) (end 49.3354 74.5034) (width 0.2) (layer "F.Cu") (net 7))
 (segment (start 88.5 81.9) (end 87.4483 81.9) (width 0.2) (layer "F.Cu") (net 7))
 (segment (start 50.4875 62.3075) (end 51.6392 62.3075) (width 0.2) (layer "F.Cu") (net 7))
 (segment (start 86.3716 80.8233) (end 87.4483 81.9) (width 0.2) (layer "F.Cu") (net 7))
 (segment (start 50.5 73.6267) (end 50.2121 73.6267) (width 0.2) (layer "F.Cu") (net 7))
 (via (at 79.3037 59.3287) (size 0.6) (drill 0.3) (layers "F.Cu" "B.Cu") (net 7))
 (segment (start 79.3037 59.3287) (end 79.3037 38.028) (width 0.2) (layer "B.Cu") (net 7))
 (segment (start 51.6514 70.1719) (end 51.6514 64.3546) (width 0.2) (layer "B.Cu") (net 7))
 (segment (start 50.5 72.475) (end 50.5 71.3233) (width 0.2) (layer "B.Cu") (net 7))
 (segment (start 50.5 71.3233) (end 51.6514 70.1719) (width 0.2) (layer "B.Cu") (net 7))
 (segment (start 50.756 63.4592) (end 50.4875 63.4592) (width 0.2) (layer "B.Cu") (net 7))
 (segment (start 50.4875 62.3075) (end 50.4875 63.4592) (width 0.2) (layer "B.Cu") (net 7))
 (segment (start 82.715 33.64) (end 82.715 34.6167) (width 0.2) (layer "B.Cu") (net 7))
 (segment (start 51.6514 64.3546) (end 50.756 63.4592) (width 0.2) (layer "B.Cu") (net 7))
 (segment (start 79.3037 38.028) (end 82.715 34.6167) (width 0.2) (layer "B.Cu") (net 7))
 (segment (start 86.0957 50.5793) (end 86.0957 43.886) (width 0.2) (layer "B.Cu") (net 15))
 (segment (start 88.88 40) (end 88.88 41.1017) (width 0.2) (layer "B.Cu") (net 15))
 (segment (start 82.715 53.96) (end 86.0957 50.5793) (width 0.2) (layer "B.Cu") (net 15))
 (segment (start 86.0957 43.886) (end 88.88 41.1017) (width 0.2) (layer "B.Cu") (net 15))
 (segment (start 89 55.295) (end 89 48) (width 0.2) (layer "B.Cu") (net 17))
 (segment (start 82.715 61.58) (end 89 55.295) (width 0.2) (layer "B.Cu") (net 17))
 (segment (start 93.5 71.5) (end 87 71.5) (width 0.2) (layer "F.Cu") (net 18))
 (segment (start 78.6983 44.4522) (end 57.3672 44.4522) (width 0.2) (layer "F.Cu") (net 18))
 (segment (start 57.3672 44.4522) (end 56.715 43.8) (width 0.2) (layer "F.Cu") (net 18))
 (via (at 78.6983 44.4522) (size 0.6) (drill 0.3) (layers "F.Cu" "B.Cu") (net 18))
 (segment (start 78.6983 61.4941) (end 78.6983 44.4522) (width 0.2) (layer "B.Cu") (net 18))
 (segment (start 82.6662 65.19) (end 82.3942 65.19) (width 0.2) (layer "B.Cu") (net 18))
 (segment (start 82.3942 65.19) (end 78.6983 61.4941) (width 0.2) (layer "B.Cu") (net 18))
 (segment (start 87 69.5238) (end 82.6662 65.19) (width 0.2) (layer "B.Cu") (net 18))
 (segment (start 87 71.5) (end 87 69.5238) (width 0.2) (layer "B.Cu") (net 18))
 (segment (start 82.3424 47.3625) (end 85.1104 47.3625) (width 0.2) (layer "F.Cu") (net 4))
 (segment (start 87.1002 49.3523) (end 97.8461 49.3523) (width 0.2) (layer "F.Cu") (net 4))
 (segment (start 78.1418 41.26) (end 81.7593 44.8775) (width 0.2) (layer "F.Cu") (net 4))
 (segment (start 81.7593 45.5374) (end 81.6788 45.6179) (width 0.2) (layer "F.Cu") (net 4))
 (segment (start 81.7593 44.8775) (end 81.7593 45.5374) (width 0.2) (layer "F.Cu") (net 4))
 (segment (start 81.6788 46.6989) (end 82.3424 47.3625) (width 0.2) (layer "F.Cu") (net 4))
 (segment (start 56.715 41.26) (end 78.1418 41.26) (width 0.2) (layer "F.Cu") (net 4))
 (segment (start 97.75 71.25) (end 104.25 71.25) (width 0.2) (layer "F.Cu") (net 4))
 (segment (start 81.6788 45.6179) (end 81.6788 46.6989) (width 0.2) (layer "F.Cu") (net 4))
 (segment (start 85.1104 47.3625) (end 87.1002 49.3523) (width 0.2) (layer "F.Cu") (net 4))
 (via (at 97.8461 49.3523) (size 0.6) (drill 0.3) (layers "F.Cu" "B.Cu") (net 4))
 (segment (start 97.8461 71.1539) (end 97.8461 49.3523) (width 0.2) (layer "B.Cu") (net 4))
 (segment (start 97.75 71.25) (end 97.8461 71.1539) (width 0.2) (layer "B.Cu") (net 4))
 (segment (start 88.9 59.5) (end 87.5983 59.5) (width 0.2) (layer "F.Cu") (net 1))
 (segment (start 82.715 59.04) (end 87.1383 59.04) (width 0.2) (layer "F.Cu") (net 1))
 (segment (start 87.1383 59.04) (end 87.5983 59.5) (width 0.2) (layer "F.Cu") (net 1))
 (segment (start 50.5 75.015) (end 51.6517 75.015) (width 0.2) (layer "F.Cu") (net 34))
 (segment (start 51.6517 75.015) (end 56.1967 70.47) (width 0.2) (layer "F.Cu") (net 34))
 (segment (start 69.0133 70.47) (end 82.715 56.7683) (width 0.2) (layer "F.Cu") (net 34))
 (segment (start 56.1967 70.47) (end 69.0133 70.47) (width 0.2) (layer "F.Cu") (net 34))
 (segment (start 82.715 56.7683) (end 82.715 56.5) (width 0.2) (layer "F.Cu") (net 34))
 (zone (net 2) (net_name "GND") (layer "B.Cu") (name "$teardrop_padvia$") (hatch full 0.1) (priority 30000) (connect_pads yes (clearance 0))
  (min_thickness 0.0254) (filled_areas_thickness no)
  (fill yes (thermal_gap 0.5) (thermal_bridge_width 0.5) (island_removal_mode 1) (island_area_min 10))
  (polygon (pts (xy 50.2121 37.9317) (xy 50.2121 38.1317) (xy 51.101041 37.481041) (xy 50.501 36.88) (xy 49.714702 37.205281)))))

